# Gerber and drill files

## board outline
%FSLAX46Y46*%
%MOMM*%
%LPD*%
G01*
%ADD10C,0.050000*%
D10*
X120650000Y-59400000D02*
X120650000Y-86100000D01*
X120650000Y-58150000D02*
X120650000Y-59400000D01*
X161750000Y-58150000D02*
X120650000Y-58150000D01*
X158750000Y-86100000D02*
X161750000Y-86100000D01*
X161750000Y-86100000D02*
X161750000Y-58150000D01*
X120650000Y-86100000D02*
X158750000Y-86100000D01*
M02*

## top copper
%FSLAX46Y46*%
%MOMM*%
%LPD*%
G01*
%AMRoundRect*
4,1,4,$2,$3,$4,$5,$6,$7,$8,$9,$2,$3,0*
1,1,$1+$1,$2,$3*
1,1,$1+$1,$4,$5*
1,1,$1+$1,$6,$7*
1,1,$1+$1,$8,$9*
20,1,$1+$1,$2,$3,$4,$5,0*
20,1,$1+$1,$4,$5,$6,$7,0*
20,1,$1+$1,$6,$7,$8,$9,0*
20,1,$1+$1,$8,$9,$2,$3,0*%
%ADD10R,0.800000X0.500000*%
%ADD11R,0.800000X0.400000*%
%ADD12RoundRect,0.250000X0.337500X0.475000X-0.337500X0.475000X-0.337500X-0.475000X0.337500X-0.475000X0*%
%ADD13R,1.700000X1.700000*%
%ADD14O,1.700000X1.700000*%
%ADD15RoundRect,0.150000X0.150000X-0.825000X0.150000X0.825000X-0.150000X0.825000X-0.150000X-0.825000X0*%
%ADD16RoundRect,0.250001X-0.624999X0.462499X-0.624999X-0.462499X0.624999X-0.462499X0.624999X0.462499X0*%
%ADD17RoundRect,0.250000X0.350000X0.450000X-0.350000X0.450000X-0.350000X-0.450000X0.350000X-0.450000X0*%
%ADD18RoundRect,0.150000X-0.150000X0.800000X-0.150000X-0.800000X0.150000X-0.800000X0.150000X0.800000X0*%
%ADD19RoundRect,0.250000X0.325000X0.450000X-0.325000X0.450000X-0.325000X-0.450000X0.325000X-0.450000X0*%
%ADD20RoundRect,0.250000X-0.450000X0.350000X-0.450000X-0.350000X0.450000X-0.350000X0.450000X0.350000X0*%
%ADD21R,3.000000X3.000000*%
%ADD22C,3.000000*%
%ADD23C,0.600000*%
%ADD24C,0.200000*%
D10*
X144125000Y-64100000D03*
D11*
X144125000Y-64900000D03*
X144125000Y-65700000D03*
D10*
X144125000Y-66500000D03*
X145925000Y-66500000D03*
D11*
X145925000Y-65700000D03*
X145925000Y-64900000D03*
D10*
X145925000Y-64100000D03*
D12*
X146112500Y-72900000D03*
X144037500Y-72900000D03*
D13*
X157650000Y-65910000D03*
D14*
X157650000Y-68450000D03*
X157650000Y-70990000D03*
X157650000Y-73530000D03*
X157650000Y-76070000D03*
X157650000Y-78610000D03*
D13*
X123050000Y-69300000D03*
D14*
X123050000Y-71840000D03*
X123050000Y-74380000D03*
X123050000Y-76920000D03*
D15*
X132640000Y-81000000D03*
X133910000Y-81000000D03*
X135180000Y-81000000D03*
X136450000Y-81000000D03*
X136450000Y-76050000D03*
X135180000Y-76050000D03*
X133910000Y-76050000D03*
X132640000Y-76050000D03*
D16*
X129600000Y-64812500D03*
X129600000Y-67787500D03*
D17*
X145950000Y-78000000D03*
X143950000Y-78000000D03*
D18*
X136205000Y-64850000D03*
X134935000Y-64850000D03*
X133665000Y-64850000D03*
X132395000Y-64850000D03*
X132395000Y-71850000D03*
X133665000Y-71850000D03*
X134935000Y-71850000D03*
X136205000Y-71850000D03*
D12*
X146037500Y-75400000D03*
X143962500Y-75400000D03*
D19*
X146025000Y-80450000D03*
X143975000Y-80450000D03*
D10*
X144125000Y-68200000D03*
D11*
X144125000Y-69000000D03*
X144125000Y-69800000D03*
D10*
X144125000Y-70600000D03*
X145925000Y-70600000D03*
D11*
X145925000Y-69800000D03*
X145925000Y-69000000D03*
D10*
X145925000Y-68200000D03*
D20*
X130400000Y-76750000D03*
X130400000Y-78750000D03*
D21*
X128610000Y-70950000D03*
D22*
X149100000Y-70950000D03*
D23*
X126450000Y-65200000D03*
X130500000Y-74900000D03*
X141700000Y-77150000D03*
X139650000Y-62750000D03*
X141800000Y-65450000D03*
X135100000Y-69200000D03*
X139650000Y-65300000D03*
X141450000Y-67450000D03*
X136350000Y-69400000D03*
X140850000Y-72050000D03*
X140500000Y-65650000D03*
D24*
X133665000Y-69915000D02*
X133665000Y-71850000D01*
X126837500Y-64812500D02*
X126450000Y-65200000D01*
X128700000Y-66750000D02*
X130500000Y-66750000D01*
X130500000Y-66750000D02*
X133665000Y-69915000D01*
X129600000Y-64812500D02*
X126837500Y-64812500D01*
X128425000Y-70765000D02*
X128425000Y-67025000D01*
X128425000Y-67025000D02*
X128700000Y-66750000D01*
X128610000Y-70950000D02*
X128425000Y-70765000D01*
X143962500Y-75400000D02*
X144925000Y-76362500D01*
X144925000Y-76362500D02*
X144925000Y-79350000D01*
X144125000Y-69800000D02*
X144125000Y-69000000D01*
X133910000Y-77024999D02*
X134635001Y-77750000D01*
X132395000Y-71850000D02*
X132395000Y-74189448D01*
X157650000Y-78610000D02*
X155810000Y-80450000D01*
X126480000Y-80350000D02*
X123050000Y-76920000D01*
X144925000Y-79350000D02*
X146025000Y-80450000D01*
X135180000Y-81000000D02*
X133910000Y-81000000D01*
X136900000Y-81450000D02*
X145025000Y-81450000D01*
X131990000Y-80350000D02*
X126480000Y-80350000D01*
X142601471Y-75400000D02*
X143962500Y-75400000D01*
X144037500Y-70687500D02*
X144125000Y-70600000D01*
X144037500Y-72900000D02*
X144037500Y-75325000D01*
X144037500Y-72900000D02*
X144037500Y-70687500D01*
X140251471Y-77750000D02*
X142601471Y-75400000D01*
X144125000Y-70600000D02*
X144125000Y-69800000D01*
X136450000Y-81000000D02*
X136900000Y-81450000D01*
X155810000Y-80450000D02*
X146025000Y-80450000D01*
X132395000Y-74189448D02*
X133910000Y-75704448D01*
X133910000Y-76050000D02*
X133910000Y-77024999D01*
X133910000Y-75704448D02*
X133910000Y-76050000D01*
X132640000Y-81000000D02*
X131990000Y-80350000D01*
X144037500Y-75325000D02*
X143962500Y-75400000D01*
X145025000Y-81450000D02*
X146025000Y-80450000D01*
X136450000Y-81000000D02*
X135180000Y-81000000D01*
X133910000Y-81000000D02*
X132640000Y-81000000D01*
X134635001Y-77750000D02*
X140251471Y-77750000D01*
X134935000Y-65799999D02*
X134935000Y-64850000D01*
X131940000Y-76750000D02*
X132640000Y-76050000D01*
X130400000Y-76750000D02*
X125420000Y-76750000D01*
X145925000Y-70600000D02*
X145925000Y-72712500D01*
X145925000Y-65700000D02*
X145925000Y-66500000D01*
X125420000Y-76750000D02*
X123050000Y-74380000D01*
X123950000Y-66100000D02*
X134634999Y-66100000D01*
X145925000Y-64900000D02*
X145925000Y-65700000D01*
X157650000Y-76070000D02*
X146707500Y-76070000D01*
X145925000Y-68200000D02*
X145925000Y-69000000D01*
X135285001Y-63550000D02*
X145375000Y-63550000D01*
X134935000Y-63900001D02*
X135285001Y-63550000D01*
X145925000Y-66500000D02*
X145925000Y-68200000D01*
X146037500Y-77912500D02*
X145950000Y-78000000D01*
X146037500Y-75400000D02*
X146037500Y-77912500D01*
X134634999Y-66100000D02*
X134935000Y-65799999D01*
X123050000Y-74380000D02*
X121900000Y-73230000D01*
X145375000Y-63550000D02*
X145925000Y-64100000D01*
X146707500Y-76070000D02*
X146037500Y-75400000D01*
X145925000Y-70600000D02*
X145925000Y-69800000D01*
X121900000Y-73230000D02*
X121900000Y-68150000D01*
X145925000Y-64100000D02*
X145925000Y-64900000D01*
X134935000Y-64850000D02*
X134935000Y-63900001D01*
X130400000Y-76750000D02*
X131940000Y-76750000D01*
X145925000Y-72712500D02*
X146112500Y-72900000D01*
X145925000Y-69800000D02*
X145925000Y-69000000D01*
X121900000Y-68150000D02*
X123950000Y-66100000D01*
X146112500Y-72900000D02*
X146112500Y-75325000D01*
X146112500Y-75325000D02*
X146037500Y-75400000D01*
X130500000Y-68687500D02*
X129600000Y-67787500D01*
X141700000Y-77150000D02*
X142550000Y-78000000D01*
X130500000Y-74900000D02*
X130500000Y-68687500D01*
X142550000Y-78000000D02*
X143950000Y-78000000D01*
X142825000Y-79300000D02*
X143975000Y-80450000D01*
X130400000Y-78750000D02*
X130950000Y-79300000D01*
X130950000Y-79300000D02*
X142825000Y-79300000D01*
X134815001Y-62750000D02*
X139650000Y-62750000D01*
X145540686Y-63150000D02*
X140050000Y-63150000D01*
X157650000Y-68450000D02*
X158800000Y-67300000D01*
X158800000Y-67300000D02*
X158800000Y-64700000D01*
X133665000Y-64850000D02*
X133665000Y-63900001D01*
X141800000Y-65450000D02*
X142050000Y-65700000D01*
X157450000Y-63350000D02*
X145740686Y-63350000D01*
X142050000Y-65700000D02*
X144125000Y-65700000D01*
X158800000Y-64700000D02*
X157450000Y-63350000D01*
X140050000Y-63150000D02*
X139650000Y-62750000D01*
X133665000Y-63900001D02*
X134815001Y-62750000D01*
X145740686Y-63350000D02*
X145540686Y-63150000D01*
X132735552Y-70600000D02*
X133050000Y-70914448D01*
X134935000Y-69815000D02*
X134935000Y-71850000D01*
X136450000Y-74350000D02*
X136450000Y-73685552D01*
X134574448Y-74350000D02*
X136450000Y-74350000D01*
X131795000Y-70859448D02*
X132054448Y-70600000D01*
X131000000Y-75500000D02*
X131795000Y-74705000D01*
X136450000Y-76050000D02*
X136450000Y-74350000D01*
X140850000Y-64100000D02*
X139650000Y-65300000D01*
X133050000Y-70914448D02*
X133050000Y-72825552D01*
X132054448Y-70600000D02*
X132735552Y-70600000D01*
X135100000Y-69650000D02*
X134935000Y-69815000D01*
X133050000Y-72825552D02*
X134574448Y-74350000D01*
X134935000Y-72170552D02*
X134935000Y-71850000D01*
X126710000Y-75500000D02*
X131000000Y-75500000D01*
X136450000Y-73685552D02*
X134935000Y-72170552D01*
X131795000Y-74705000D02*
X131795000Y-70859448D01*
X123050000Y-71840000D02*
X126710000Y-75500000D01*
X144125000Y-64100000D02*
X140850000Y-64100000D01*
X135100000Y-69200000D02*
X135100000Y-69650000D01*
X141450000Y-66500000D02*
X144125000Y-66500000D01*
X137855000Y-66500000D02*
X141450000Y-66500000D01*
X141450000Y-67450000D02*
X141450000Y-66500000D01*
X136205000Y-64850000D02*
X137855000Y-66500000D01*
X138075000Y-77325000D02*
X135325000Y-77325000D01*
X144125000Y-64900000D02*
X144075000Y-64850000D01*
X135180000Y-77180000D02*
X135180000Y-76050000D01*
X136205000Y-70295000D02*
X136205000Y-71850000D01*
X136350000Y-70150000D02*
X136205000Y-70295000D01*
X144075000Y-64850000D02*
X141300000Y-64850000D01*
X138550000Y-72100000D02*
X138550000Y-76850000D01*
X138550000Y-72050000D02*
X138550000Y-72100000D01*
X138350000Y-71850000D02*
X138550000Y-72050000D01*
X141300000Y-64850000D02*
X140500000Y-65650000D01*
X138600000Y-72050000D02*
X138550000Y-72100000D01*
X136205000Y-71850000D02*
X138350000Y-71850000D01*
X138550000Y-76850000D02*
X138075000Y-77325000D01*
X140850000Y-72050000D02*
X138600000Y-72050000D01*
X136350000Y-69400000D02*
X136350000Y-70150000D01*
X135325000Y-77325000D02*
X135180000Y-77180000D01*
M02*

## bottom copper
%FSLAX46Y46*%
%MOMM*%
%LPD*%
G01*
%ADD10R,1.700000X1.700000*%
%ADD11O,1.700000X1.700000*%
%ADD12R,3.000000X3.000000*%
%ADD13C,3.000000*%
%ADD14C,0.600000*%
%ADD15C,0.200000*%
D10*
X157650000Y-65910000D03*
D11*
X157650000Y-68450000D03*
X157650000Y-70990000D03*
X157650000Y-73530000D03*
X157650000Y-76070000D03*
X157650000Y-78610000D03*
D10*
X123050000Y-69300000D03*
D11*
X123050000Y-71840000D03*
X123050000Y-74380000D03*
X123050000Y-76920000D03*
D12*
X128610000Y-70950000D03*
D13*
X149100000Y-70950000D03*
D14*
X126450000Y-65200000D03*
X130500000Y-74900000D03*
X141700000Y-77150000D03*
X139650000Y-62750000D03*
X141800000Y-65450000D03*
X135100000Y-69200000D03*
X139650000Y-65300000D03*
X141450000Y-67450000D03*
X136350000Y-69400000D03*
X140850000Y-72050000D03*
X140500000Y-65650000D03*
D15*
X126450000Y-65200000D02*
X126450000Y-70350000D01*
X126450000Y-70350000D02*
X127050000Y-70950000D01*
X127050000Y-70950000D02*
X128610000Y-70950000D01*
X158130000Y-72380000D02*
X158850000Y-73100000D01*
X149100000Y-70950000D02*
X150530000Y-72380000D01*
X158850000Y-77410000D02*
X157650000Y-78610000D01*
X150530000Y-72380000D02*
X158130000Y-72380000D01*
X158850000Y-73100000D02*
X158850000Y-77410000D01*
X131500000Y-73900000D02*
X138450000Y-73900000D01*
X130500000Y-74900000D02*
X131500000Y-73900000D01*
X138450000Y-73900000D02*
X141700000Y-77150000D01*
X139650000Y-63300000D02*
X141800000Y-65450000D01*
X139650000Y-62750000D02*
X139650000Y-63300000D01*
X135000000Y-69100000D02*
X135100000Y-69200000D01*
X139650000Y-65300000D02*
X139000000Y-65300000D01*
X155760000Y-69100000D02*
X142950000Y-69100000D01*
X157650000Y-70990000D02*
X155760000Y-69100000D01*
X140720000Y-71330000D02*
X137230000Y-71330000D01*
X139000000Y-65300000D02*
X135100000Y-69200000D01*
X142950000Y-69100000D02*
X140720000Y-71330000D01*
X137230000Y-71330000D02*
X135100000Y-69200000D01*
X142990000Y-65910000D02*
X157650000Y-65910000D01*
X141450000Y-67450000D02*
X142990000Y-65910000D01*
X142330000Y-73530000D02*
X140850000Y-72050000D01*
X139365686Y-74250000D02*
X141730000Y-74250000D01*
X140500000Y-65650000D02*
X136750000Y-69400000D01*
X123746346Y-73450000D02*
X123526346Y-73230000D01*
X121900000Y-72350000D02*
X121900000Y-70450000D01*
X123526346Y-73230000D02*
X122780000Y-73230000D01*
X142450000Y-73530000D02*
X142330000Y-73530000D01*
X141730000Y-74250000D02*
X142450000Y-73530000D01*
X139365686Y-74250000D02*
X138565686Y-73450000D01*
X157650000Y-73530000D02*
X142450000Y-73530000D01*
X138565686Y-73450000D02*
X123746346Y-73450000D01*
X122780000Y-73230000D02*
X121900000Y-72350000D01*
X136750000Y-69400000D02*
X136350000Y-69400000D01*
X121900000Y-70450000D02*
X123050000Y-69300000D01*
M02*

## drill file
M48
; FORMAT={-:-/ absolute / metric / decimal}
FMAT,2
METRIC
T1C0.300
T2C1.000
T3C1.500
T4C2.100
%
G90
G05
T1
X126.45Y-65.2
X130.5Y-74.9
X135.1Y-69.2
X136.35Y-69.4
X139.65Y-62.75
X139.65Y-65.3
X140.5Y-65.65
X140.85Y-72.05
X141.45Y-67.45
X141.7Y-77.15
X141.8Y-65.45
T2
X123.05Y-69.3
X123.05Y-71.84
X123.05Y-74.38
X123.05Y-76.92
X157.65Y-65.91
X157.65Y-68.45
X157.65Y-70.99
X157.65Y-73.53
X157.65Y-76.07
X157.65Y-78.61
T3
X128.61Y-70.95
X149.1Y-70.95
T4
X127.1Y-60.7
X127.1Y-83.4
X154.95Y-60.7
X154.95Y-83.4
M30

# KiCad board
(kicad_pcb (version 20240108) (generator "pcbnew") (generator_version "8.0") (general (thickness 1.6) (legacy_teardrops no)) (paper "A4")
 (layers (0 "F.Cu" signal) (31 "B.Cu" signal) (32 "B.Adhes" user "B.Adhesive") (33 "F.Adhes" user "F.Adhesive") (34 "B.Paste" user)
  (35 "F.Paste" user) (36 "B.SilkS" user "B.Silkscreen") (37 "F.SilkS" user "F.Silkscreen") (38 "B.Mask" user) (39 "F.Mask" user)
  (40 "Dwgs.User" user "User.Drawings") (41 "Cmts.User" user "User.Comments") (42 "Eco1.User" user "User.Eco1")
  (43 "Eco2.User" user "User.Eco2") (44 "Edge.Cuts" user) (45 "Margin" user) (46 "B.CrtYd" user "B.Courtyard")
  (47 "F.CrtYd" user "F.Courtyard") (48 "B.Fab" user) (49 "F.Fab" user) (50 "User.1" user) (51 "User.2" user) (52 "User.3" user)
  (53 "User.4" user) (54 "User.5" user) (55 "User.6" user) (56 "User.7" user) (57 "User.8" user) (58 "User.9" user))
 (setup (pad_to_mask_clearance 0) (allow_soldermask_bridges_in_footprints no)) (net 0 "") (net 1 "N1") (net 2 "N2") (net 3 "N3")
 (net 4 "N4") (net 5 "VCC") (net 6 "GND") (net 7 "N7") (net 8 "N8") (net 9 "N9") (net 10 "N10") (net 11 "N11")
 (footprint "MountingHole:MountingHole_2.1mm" (layer "F.Cu") (at 127.1 60.7)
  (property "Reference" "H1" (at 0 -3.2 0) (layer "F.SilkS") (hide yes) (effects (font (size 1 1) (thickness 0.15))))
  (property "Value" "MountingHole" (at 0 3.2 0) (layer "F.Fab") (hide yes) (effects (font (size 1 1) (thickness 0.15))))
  (pad "" np_thru_hole circle (at 0 0) (size 2.1 2.1) (drill 2.1) (layers "*.Cu" "*.Mask")))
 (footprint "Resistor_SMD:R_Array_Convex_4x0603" (layer "F.Cu") (at 145.025 65.3)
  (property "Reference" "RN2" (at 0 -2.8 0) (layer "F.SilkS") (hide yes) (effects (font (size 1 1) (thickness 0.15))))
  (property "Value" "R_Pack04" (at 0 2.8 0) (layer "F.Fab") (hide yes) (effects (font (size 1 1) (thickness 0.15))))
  (pad "1" smd rect (at -0.9 -1.2) (size 0.8 0.5) (layers "F.Cu" "F.Paste" "F.Mask") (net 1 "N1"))
  (pad "2" smd rect (at -0.9 -0.4) (size 0.8 0.4) (layers "F.Cu" "F.Paste" "F.Mask") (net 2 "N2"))
  (pad "3" smd rect (at -0.9 0.4) (size 0.8 0.4) (layers "F.Cu" "F.Paste" "F.Mask") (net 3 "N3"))
  (pad "4" smd rect (at -0.9 1.2) (size 0.8 0.5) (layers "F.Cu" "F.Paste" "F.Mask") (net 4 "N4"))
  (pad "5" smd rect (at 0.9 1.2) (size 0.8 0.5) (layers "F.Cu" "F.Paste" "F.Mask") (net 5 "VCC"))
  (pad "6" smd rect (at 0.9 0.4) (size 0.8 0.4) (layers "F.Cu" "F.Paste" "F.Mask") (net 5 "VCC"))
  (pad "7" smd rect (at 0.9 -0.4) (size 0.8 0.4) (layers "F.Cu" "F.Paste" "F.Mask") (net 5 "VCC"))
  (pad "8" smd rect (at 0.9 -1.2) (size 0.8 0.5) (layers "F.Cu" "F.Paste" "F.Mask") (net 5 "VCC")))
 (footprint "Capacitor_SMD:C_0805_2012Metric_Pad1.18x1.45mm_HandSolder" (layer "F.Cu") (at 145.075 72.9 180)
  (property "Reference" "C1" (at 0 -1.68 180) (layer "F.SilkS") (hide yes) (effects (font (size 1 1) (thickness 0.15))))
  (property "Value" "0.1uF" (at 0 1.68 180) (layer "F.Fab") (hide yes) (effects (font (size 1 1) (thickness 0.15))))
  (pad "1" smd roundrect (at -1.0375 0 180) (size 1.175 1.45) (layers "F.Cu" "F.Paste" "F.Mask") (roundrect_rratio 0.212766) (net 5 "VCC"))
  (pad "2" smd roundrect (at 1.0375 0 180) (size 1.175 1.45) (layers "F.Cu" "F.Paste" "F.Mask") (roundrect_rratio 0.212766) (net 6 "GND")))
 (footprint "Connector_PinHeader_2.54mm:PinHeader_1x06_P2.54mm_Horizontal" (layer "F.Cu") (at 157.65 65.91)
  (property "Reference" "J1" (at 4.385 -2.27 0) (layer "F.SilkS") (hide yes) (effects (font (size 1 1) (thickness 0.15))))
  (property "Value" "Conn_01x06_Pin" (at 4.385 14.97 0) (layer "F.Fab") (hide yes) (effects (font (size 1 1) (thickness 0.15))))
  (pad "1" thru_hole rect (at 0 0) (size 1.7 1.7) (drill 1) (layers "*.Cu" "*.Mask") (remove_unused_layers no) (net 4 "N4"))
  (pad "2" thru_hole oval (at 0 2.54) (size 1.7 1.7) (drill 1) (layers "*.Cu" "*.Mask") (remove_unused_layers no) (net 3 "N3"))
  (pad "3" thru_hole oval (at 0 5.08) (size 1.7 1.7) (drill 1) (layers "*.Cu" "*.Mask") (remove_unused_layers no) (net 1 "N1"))
  (pad "4" thru_hole oval (at 0 7.62) (size 1.7 1.7) (drill 1) (layers "*.Cu" "*.Mask") (remove_unused_layers no) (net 2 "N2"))
  (pad "5" thru_hole oval (at 0 10.16) (size 1.7 1.7) (drill 1) (layers "*.Cu" "*.Mask") (remove_unused_layers no) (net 5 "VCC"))
  (pad "6" thru_hole oval (at 0 12.7) (size 1.7 1.7) (drill 1) (layers "*.Cu" "*.Mask") (remove_unused_layers no) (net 6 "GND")))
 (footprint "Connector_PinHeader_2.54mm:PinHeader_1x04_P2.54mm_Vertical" (layer "F.Cu") (at 123.05 69.3)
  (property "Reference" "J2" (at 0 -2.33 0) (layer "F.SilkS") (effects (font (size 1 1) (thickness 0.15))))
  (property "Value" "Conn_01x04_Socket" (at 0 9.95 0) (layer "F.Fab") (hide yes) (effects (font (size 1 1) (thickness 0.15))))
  (pad "1" thru_hole rect (at 0 0) (size 1.7 1.7) (drill 1) (layers "*.Cu" "*.Mask") (remove_unused_layers no) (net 2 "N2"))
  (pad "2" thru_hole oval (at 0 2.54) (size 1.7 1.7) (drill 1) (layers "*.Cu" "*.Mask") (remove_unused_layers no) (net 1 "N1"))
  (pad "3" thru_hole oval (at 0 5.08) (size 1.7 1.7) (drill 1) (layers "*.Cu" "*.Mask") (remove_unused_layers no) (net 5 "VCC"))
  (pad "4" thru_hole oval (at 0 7.62) (size 1.7 1.7) (drill 1) (layers "*.Cu" "*.Mask") (remove_unused_layers no) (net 6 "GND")))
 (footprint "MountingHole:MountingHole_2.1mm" (layer "F.Cu") (at 154.95 60.7)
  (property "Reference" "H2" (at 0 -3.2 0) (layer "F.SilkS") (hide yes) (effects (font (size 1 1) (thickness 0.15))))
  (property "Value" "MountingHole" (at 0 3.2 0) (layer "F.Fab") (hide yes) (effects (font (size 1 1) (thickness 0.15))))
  (pad "" np_thru_hole circle (at 0 0) (size 2.1 2.1) (drill 2.1) (layers "*.Cu" "*.Mask")))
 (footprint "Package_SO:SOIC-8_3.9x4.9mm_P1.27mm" (layer "F.Cu") (at 134.545 78.525 90)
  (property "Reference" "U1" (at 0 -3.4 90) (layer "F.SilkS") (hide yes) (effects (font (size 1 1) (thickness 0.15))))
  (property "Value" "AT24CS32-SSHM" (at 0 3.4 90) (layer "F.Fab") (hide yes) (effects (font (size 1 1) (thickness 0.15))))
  (pad "1" smd roundrect (at -2.475 -1.905 90) (size 1.95 0.6) (layers "F.Cu" "F.Paste" "F.Mask") (roundrect_rratio 0.25) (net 6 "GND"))
  (pad "2" smd roundrect (at -2.475 -0.635 90) (size 1.95 0.6) (layers "F.Cu" "F.Paste" "F.Mask") (roundrect_rratio 0.25) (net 6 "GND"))
  (pad "3" smd roundrect (at -2.475 0.635 90) (size 1.95 0.6) (layers "F.Cu" "F.Paste" "F.Mask") (roundrect_rratio 0.25) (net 6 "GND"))
  (pad "4" smd roundrect (at -2.475 1.905 90) (size 1.95 0.6) (layers "F.Cu" "F.Paste" "F.Mask") (roundrect_rratio 0.25) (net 6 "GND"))
  (pad "5" smd roundrect (at 2.475 1.905 90) (size 1.95 0.6) (layers "F.Cu" "F.Paste" "F.Mask") (roundrect_rratio 0.25) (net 1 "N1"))
  (pad "6" smd roundrect (at 2.475 0.635 90) (size 1.95 0.6) (layers "F.Cu" "F.Paste" "F.Mask") (roundrect_rratio 0.25) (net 2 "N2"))
  (pad "7" smd roundrect (at 2.475 -0.635 90) (size 1.95 0.6) (layers "F.Cu" "F.Paste" "F.Mask") (roundrect_rratio 0.25) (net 6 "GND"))
  (pad "8" smd roundrect (at 2.475 -1.905 90) (size 1.95 0.6) (layers "F.Cu" "F.Paste" "F.Mask") (roundrect_rratio 0.25) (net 5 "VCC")))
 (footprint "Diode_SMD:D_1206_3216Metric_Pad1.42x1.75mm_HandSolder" (layer "F.Cu") (at 129.6 66.3 -90)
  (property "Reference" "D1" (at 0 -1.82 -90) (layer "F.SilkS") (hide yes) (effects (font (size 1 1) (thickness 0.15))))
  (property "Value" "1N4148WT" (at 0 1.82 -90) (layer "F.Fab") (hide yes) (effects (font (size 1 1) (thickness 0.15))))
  (pad "1" smd roundrect (at -1.4875 0 270) (size 1.425 1.75) (layers "F.Cu" "F.Paste" "F.Mask") (roundrect_rratio 0.175439) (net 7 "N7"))
  (pad "2" smd roundrect (at 1.4875 0 270) (size 1.425 1.75) (layers "F.Cu" "F.Paste" "F.Mask") (roundrect_rratio 0.175439) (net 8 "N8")))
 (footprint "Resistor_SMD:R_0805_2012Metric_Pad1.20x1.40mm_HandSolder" (layer "F.Cu") (at 144.95 78 180)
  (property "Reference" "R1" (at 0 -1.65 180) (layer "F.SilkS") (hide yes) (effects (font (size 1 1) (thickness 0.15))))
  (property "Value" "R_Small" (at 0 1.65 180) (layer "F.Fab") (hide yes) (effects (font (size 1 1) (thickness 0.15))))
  (pad "1" smd roundrect (at -1 0 180) (size 1.2 1.4) (layers "F.Cu" "F.Paste" "F.Mask") (roundrect_rratio 0.208333) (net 5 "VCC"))
  (pad "2" smd roundrect (at 1 0 180) (size 1.2 1.4) (layers "F.Cu" "F.Paste" "F.Mask") (roundrect_rratio 0.208333) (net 8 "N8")))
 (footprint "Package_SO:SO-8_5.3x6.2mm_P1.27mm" (layer "F.Cu") (at 134.3 68.35 -90)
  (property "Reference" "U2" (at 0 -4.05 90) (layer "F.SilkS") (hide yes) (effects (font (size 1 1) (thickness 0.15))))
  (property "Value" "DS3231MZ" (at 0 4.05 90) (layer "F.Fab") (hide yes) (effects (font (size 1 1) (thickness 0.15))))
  (pad "1" smd roundrect (at -3.5 -1.905 270) (size 1.9 0.6) (layers "F.Cu" "F.Paste" "F.Mask") (roundrect_rratio 0.25) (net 4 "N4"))
  (pad "2" smd roundrect (at -3.5 -0.635 270) (size 1.9 0.6) (layers "F.Cu" "F.Paste" "F.Mask") (roundrect_rratio 0.25) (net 5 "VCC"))
  (pad "3" smd roundrect (at -3.5 0.635 270) (size 1.9 0.6) (layers "F.Cu" "F.Paste" "F.Mask") (roundrect_rratio 0.25) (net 3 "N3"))
  (pad "4" smd roundrect (at -3.5 1.905 270) (size 1.9 0.6) (layers "F.Cu" "F.Paste" "F.Mask") (roundrect_rratio 0.25) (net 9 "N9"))
  (pad "5" smd roundrect (at 3.5 1.905 270) (size 1.9 0.6) (layers "F.Cu" "F.Paste" "F.Mask") (roundrect_rratio 0.25) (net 6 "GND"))
  (pad "6" smd roundrect (at 3.5 0.635 270) (size 1.9 0.6) (layers "F.Cu" "F.Paste" "F.Mask") (roundrect_rratio 0.25) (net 7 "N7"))
  (pad "7" smd roundrect (at 3.5 -0.635 270) (size 1.9 0.6) (layers "F.Cu" "F.Paste" "F.Mask") (roundrect_rratio 0.25) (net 1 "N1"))
  (pad "8" smd roundrect (at 3.5 -1.905 270) (size 1.9 0.6) (layers "F.Cu" "F.Paste" "F.Mask") (roundrect_rratio 0.25) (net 2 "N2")))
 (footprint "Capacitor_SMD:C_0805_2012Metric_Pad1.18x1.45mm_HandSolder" (layer "F.Cu") (at 145 75.4 180)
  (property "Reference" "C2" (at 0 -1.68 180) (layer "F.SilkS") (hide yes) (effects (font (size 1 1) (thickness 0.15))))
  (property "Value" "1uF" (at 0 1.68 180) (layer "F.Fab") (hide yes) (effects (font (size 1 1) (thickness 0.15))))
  (pad "1" smd roundrect (at -1.0375 0 180) (size 1.175 1.45) (layers "F.Cu" "F.Paste" "F.Mask") (roundrect_rratio 0.212766) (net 5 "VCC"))
  (pad "2" smd roundrect (at 1.0375 0 180) (size 1.175 1.45) (layers "F.Cu" "F.Paste" "F.Mask") (roundrect_rratio 0.212766) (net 6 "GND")))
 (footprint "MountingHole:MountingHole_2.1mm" (layer "F.Cu") (at 154.95 83.4)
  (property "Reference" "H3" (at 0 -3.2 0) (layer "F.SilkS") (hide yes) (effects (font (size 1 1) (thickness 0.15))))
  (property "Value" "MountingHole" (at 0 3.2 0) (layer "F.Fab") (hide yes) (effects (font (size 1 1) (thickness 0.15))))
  (pad "" np_thru_hole circle (at 0 0) (size 2.1 2.1) (drill 2.1) (layers "*.Cu" "*.Mask")))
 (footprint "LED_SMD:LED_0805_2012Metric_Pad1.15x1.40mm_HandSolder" (layer "F.Cu") (at 145 80.45 180)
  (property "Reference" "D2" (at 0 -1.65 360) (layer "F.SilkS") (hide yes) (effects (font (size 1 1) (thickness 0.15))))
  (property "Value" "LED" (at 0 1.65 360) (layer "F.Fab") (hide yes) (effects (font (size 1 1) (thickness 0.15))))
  (pad "1" smd roundrect (at -1.025 0 180) (size 1.15 1.4) (layers "F.Cu" "F.Paste" "F.Mask") (roundrect_rratio 0.217391) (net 6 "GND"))
  (pad "2" smd roundrect (at 1.025 0 180) (size 1.15 1.4) (layers "F.Cu" "F.Paste" "F.Mask") (roundrect_rratio 0.217391) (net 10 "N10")))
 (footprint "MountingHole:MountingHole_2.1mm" (layer "F.Cu") (at 127.1 83.4)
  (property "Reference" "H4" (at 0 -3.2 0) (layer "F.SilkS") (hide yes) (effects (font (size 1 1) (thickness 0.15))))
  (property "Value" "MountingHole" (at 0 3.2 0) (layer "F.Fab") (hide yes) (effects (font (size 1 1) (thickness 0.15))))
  (pad "" np_thru_hole circle (at 0 0) (size 2.1 2.1) (drill 2.1) (layers "*.Cu" "*.Mask")))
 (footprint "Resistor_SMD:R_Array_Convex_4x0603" (layer "F.Cu") (at 145.025 69.4)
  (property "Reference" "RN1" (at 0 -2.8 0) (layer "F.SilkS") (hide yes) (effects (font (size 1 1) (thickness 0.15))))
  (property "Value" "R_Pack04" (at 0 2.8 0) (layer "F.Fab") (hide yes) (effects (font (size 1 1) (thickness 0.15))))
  (pad "1" smd rect (at -0.9 -1.2) (size 0.8 0.5) (layers "F.Cu" "F.Paste" "F.Mask") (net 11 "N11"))
  (pad "2" smd rect (at -0.9 -0.4) (size 0.8 0.4) (layers "F.Cu" "F.Paste" "F.Mask") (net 6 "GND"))
  (pad "3" smd rect (at -0.9 0.4) (size 0.8 0.4) (layers "F.Cu" "F.Paste" "F.Mask") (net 6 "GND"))
  (pad "4" smd rect (at -0.9 1.2) (size 0.8 0.5) (layers "F.Cu" "F.Paste" "F.Mask") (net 6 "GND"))
  (pad "5" smd rect (at 0.9 1.2) (size 0.8 0.5) (layers "F.Cu" "F.Paste" "F.Mask") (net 5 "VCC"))
  (pad "6" smd rect (at 0.9 0.4) (size 0.8 0.4) (layers "F.Cu" "F.Paste" "F.Mask") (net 5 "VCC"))
  (pad "7" smd rect (at 0.9 -0.4) (size 0.8 0.4) (layers "F.Cu" "F.Paste" "F.Mask") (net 5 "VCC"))
  (pad "8" smd rect (at 0.9 -1.2) (size 0.8 0.5) (layers "F.Cu" "F.Paste" "F.Mask") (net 5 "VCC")))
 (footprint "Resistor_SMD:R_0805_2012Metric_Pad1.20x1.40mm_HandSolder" (layer "F.Cu") (at 130.4 77.75 -90)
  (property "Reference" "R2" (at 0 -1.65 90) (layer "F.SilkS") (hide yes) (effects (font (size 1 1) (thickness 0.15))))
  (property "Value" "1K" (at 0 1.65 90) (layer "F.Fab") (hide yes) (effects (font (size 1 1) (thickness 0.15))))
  (pad "1" smd roundrect (at -1 0 270) (size 1.2 1.4) (layers "F.Cu" "F.Paste" "F.Mask") (roundrect_rratio 0.208333) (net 5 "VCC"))
  (pad "2" smd roundrect (at 1 0 270) (size 1.2 1.4) (layers "F.Cu" "F.Paste" "F.Mask") (roundrect_rratio 0.208333) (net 10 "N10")))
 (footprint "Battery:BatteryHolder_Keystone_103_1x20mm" (layer "B.Cu") (at 128.61 70.95)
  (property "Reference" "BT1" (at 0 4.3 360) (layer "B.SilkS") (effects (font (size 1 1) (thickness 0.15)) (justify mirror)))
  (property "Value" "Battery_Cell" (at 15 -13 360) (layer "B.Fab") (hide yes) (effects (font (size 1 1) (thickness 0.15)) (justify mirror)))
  (pad "1" thru_hole rect (at 0 0) (size 3 3) (drill 1.5) (layers "*.Cu" "*.Mask") (remove_unused_layers no) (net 7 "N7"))
  (pad "2" thru_hole circle (at 20.49 0) (size 3 3) (drill 1.5) (layers "*.Cu" "*.Mask") (remove_unused_layers no) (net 6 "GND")))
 (gr_line (start 120.65 59.4) (end 120.65 86.1) (stroke (width 0.05) (type default)) (layer "Edge.Cuts"))
 (gr_line (start 120.65 58.15) (end 120.65 59.4) (stroke (width 0.05) (type default)) (layer "Edge.Cuts"))
 (gr_line (start 161.75 58.15) (end 120.65 58.15) (stroke (width 0.05) (type default)) (layer "Edge.Cuts"))
 (gr_line (start 158.75 86.1) (end 161.75 86.1) (stroke (width 0.05) (type default)) (layer "Edge.Cuts"))
 (gr_line (start 161.75 86.1) (end 161.75 58.15) (stroke (width 0.05) (type default)) (layer "Edge.Cuts"))
 (gr_line (start 120.65 86.1) (end 158.75 86.1) (stroke (width 0.05) (type default)) (layer "Edge.Cuts"))
 (segment (start 133.665 69.915) (end 133.665 71.85) (width 0.2) (layer "F.Cu") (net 7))
 (segment (start 126.8375 64.8125) (end 126.45 65.2) (width 0.2) (layer "F.Cu") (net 7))
 (segment (start 128.7 66.75) (end 130.5 66.75) (width 0.2) (layer "F.Cu") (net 7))
 (segment (start 130.5 66.75) (end 133.665 69.915) (width 0.2) (layer "F.Cu") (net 7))
 (segment (start 129.6 64.8125) (end 126.8375 64.8125) (width 0.2) (layer "F.Cu") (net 7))
 (segment (start 128.425 70.765) (end 128.425 67.025) (width 0.2) (layer "F.Cu") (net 7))
 (segment (start 128.425 67.025) (end 128.7 66.75) (width 0.2) (layer "F.Cu") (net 7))
 (segment (start 128.61 70.95) (end 128.425 70.765) (width 0.2) (layer "F.Cu") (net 7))
 (via (at 126.45 65.2) (size 0.6) (drill 0.3) (layers "F.Cu" "B.Cu") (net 7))
 (segment (start 126.45 65.2) (end 126.45 70.35) (width 0.2) (layer "B.Cu") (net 7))
 (segment (start 126.45 70.35) (end 127.05 70.95) (width 0.2) (layer "B.Cu") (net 7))
 (segment (start 127.05 70.95) (end 128.61 70.95) (width 0.2) (layer "B.Cu") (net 7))
 (segment (start 143.9625 75.4) (end 144.925 76.3625) (width 0.2) (layer "F.Cu") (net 6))
 (segment (start 144.925 76.3625) (end 144.925 79.35) (width 0.2) (layer "F.Cu") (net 6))
 (segment (start 144.125 69.8) (end 144.125 69) (width 0.2) (layer "F.Cu") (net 6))
 (segment (start 133.91 77.024999) (end 134.635001 77.75) (width 0.2) (layer "F.Cu") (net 6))
 (segment (start 132.395 71.85) (end 132.395 74.189448) (width 0.2) (layer "F.Cu") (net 6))
 (segment (start 157.65 78.61) (end 155.81 80.45) (width 0.2) (layer "F.Cu") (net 6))
 (segment (start 126.48 80.35) (end 123.05 76.92) (width 0.2) (layer "F.Cu") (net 6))
 (segment (start 144.925 79.35) (end 146.025 80.45) (width 0.2) (layer "F.Cu") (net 6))
 (segment (start 135.18 81) (end 133.91 81) (width 0.2) (layer "F.Cu") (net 6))
 (segment (start 136.9 81.45) (end 145.025 81.45) (width 0.2) (layer "F.Cu") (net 6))
 (segment (start 131.99 80.35) (end 126.48 80.35) (width 0.2) (layer "F.Cu") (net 6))
 (segment (start 142.601471 75.4) (end 143.9625 75.4) (width 0.2) (layer "F.Cu") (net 6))
 (segment (start 144.0375 70.6875) (end 144.125 70.6) (width 0.2) (layer "F.Cu") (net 6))
 (segment (start 144.0375 72.9) (end 144.0375 75.325) (width 0.2) (layer "F.Cu") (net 6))
 (segment (start 144.0375 72.9) (end 144.0375 70.6875) (width 0.2) (layer "F.Cu") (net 6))
 (segment (start 140.251471 77.75) (end 142.601471 75.4) (width 0.2) (layer "F.Cu") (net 6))
 (segment (start 144.125 70.6) (end 144.125 69.8) (width 0.2) (layer "F.Cu") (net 6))
 (segment (start 136.45 81) (end 136.9 81.45) (width 0.2) (layer "F.Cu") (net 6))
 (segment (start 155.81 80.45) (end 146.025 80.45) (width 0.2) (layer "F.Cu") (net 6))
 (segment (start 132.395 74.189448) (end 133.91 75.704448) (width 0.2) (layer "F.Cu") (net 6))
 (segment (start 133.91 76.05) (end 133.91 77.024999) (width 0.2) (layer "F.Cu") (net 6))
 (segment (start 133.91 75.704448) (end 133.91 76.05) (width 0.2) (layer "F.Cu") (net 6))
 (segment (start 132.64 81) (end 131.99 80.35) (width 0.2) (layer "F.Cu") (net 6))
 (segment (start 144.0375 75.325) (end 143.9625 75.4) (width 0.2) (layer "F.Cu") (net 6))
 (segment (start 145.025 81.45) (end 146.025 80.45) (width 0.2) (layer "F.Cu") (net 6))
 (segment (start 136.45 81) (end 135.18 81) (width 0.2) (layer "F.Cu") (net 6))
 (segment (start 133.91 81) (end 132.64 81) (width 0.2) (layer "F.Cu") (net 6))
 (segment (start 134.635001 77.75) (end 140.251471 77.75) (width 0.2) (layer "F.Cu") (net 6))
 (segment (start 158.13 72.38) (end 158.85 73.1) (width 0.2) (layer "B.Cu") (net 6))
 (segment (start 149.1 70.95) (end 150.53 72.38) (width 0.2) (layer "B.Cu") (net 6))
 (segment (start 158.85 77.41) (end 157.65 78.61) (width 0.2) (layer "B.Cu") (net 6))
 (segment (start 150.53 72.38) (end 158.13 72.38) (width 0.2) (layer "B.Cu") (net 6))
 (segment (start 158.85 73.1) (end 158.85 77.41) (width 0.2) (layer "B.Cu") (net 6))
 (segment (start 134.935 65.799999) (end 134.935 64.85) (width 0.2) (layer "F.Cu") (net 5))
 (segment (start 131.94 76.75) (end 132.64 76.05) (width 0.2) (layer "F.Cu") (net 5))
 (segment (start 130.4 76.75) (end 125.42 76.75) (width 0.2) (layer "F.Cu") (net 5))
 (segment (start 145.925 70.6) (end 145.925 72.7125) (width 0.2) (layer "F.Cu") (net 5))
 (segment (start 145.925 65.7) (end 145.925 66.5) (width 0.2) (layer "F.Cu") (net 5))
 (segment (start 125.42 76.75) (end 123.05 74.38) (width 0.2) (layer "F.Cu") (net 5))
 (segment (start 123.95 66.1) (end 134.634999 66.1) (width 0.2) (layer "F.Cu") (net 5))
 (segment (start 145.925 64.9) (end 145.925 65.7) (width 0.2) (layer "F.Cu") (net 5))
 (segment (start 157.65 76.07) (end 146.7075 76.07) (width 0.2) (layer "F.Cu") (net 5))
 (segment (start 145.925 68.2) (end 145.925 69) (width 0.2) (layer "F.Cu") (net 5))
 (segment (start 135.285001 63.55) (end 145.375 63.55) (width 0.2) (layer "F.Cu") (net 5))
 (segment (start 134.935 63.900001) (end 135.285001 63.55) (width 0.2) (layer "F.Cu") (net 5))
 (segment (start 145.925 66.5) (end 145.925 68.2) (width 0.2) (layer "F.Cu") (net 5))
 (segment (start 146.0375 77.9125) (end 145.95 78) (width 0.2) (layer "F.Cu") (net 5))
 (segment (start 146.0375 75.4) (end 146.0375 77.9125) (width 0.2) (layer "F.Cu") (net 5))
 (segment (start 134.634999 66.1) (end 134.935 65.799999) (width 0.2) (layer "F.Cu") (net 5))
 (segment (start 123.05 74.38) (end 121.9 73.23) (width 0.2) (layer "F.Cu") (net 5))
 (segment (start 145.375 63.55) (end 145.925 64.1) (width 0.2) (layer "F.Cu") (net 5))
 (segment (start 146.7075 76.07) (end 146.0375 75.4) (width 0.2) (layer "F.Cu") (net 5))
 (segment (start 145.925 70.6) (end 145.925 69.8) (width 0.2) (layer "F.Cu") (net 5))
 (segment (start 121.9 73.23) (end 121.9 68.15) (width 0.2) (layer "F.Cu") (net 5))
 (segment (start 145.925 64.1) (end 145.925 64.9) (width 0.2) (layer "F.Cu") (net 5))
 (segment (start 134.935 64.85) (end 134.935 63.900001) (width 0.2) (layer "F.Cu") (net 5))
 (segment (start 130.4 76.75) (end 131.94 76.75) (width 0.2) (layer "F.Cu") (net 5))
 (segment (start 145.925 72.7125) (end 146.1125 72.9) (width 0.2) (layer "F.Cu") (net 5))
 (segment (start 145.925 69.8) (end 145.925 69) (width 0.2) (layer "F.Cu") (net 5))
 (segment (start 121.9 68.15) (end 123.95 66.1) (width 0.2) (layer "F.Cu") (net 5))
 (segment (start 146.1125 72.9) (end 146.1125 75.325) (width 0.2) (layer "F.Cu") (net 5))
 (segment (start 146.1125 75.325) (end 146.0375 75.4) (width 0.2) (layer "F.Cu") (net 5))
 (segment (start 130.5 68.6875) (end 129.6 67.7875) (width 0.2) (layer "F.Cu") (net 8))
 (segment (start 141.7 77.15) (end 142.55 78) (width 0.2) (layer "F.Cu") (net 8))
 (segment (start 130.5 74.9) (end 130.5 68.6875) (width 0.2) (layer "F.Cu") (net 8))
 (segment (start 142.55 78) (end 143.95 78) (width 0.2) (layer "F.Cu") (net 8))
 (via (at 130.5 74.9) (size 0.6) (drill 0.3) (layers "F.Cu" "B.Cu") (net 8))
 (via (at 141.7 77.15) (size 0.6) (drill 0.3) (layers "F.Cu" "B.Cu") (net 8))
 (segment (start 131.5 73.9) (end 138.45 73.9) (width 0.2) (layer "B.Cu") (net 8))
 (segment (start 130.5 74.9) (end 131.5 73.9) (width 0.2) (layer "B.Cu") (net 8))
 (segment (start 138.45 73.9) (end 141.7 77.15) (width 0.2) (layer "B.Cu") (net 8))
 (segment (start 142.825 79.3) (end 143.975 80.45) (width 0.2) (layer "F.Cu") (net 10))
 (segment (start 130.4 78.75) (end 130.95 79.3) (width 0.2) (layer "F.Cu") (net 10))
 (segment (start 130.95 79.3) (end 142.825 79.3) (width 0.2) (layer "F.Cu") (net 10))
 (segment (start 134.815001 62.75) (end 139.65 62.75) (width 0.2) (layer "F.Cu") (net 3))
 (segment (start 145.540686 63.15) (end 140.05 63.15) (width 0.2) (layer "F.Cu") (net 3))
 (segment (start 157.65 68.45) (end 158.8 67.3) (width 0.2) (layer "F.Cu") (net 3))
 (segment (start 158.8 67.3) (end 158.8 64.7) (width 0.2) (layer "F.Cu") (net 3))
 (segment (start 133.665 64.85) (end 133.665 63.900001) (width 0.2) (layer "F.Cu") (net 3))
 (segment (start 141.8 65.45) (end 142.05 65.7) (width 0.2) (layer "F.Cu") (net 3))
 (segment (start 157.45 63.35) (end 145.740686 63.35) (width 0.2) (layer "F.Cu") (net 3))
 (segment (start 142.05 65.7) (end 144.125 65.7) (width 0.2) (layer "F.Cu") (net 3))
 (segment (start 158.8 64.7) (end 157.45 63.35) (width 0.2) (layer "F.Cu") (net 3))
 (segment (start 140.05 63.15) (end 139.65 62.75) (width 0.2) (layer "F.Cu") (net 3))
 (segment (start 133.665 63.900001) (end 134.815001 62.75) (width 0.2) (layer "F.Cu") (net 3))
 (segment (start 145.740686 63.35) (end 145.540686 63.15) (width 0.2) (layer "F.Cu") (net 3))
 (via (at 139.65 62.75) (size 0.6) (drill 0.3) (layers "F.Cu" "B.Cu") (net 3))
 (via (at 141.8 65.45) (size 0.6) (drill 0.3) (layers "F.Cu" "B.Cu") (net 3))
 (segment (start 139.65 63.3) (end 141.8 65.45) (width 0.2) (layer "B.Cu") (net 3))
 (segment (start 139.65 62.75) (end 139.65 63.3) (width 0.2) (layer "B.Cu") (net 3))
 (segment (start 132.735552 70.6) (end 133.05 70.914448) (width 0.2) (layer "F.Cu") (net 1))
 (segment (start 134.935 69.815) (end 134.935 71.85) (width 0.2) (layer "F.Cu") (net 1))
 (segment (start 136.45 74.35) (end 136.45 73.685552) (width 0.2) (layer "F.Cu") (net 1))
 (segment (start 134.574448 74.35) (end 136.45 74.35) (width 0.2) (layer "F.Cu") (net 1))
 (segment (start 131.795 70.859448) (end 132.054448 70.6) (width 0.2) (layer "F.Cu") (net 1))
 (segment (start 131 75.5) (end 131.795 74.705) (width 0.2) (layer "F.Cu") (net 1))
 (segment (start 136.45 76.05) (end 136.45 74.35) (width 0.2) (layer "F.Cu") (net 1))
 (segment (start 140.85 64.1) (end 139.65 65.3) (width 0.2) (layer "F.Cu") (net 1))
 (segment (start 133.05 70.914448) (end 133.05 72.825552) (width 0.2) (layer "F.Cu") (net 1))
 (segment (start 132.054448 70.6) (end 132.735552 70.6) (width 0.2) (layer "F.Cu") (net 1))
 (segment (start 135.1 69.65) (end 134.935 69.815) (width 0.2) (layer "F.Cu") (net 1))
 (segment (start 133.05 72.825552) (end 134.574448 74.35) (width 0.2) (layer "F.Cu") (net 1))
 (segment (start 134.935 72.170552) (end 134.935 71.85) (width 0.2) (layer "F.Cu") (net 1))
 (segment (start 126.71 75.5) (end 131 75.5) (width 0.2) (layer "F.Cu") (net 1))
 (segment (start 136.45 73.685552) (end 134.935 72.170552) (width 0.2) (layer "F.Cu") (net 1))
 (segment (start 131.795 74.705) (end 131.795 70.859448) (width 0.2) (layer "F.Cu") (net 1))
 (segment (start 123.05 71.84) (end 126.71 75.5) (width 0.2) (layer "F.Cu") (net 1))
 (segment (start 144.125 64.1) (end 140.85 64.1) (width 0.2) (layer "F.Cu") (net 1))
 (segment (start 135.1 69.2) (end 135.1 69.65) (width 0.2) (layer "F.Cu") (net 1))
 (via (at 135.1 69.2) (size 0.6) (drill 0.3) (layers "F.Cu" "B.Cu") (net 1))
 (via (at 139.65 65.3) (size 0.6) (drill 0.3) (layers "F.Cu" "B.Cu") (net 1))
 (segment (start 135 69.1) (end 135.1 69.2) (width 0.2) (layer "B.Cu") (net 1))
 (segment (start 139.65 65.3) (end 139 65.3) (width 0.2) (layer "B.Cu") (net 1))
 (segment (start 155.76 69.1) (end 142.95 69.1) (width 0.2) (layer "B.Cu") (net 1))
 (segment (start 157.65 70.99) (end 155.76 69.1) (width 0.2) (layer "B.Cu") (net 1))
 (segment (start 140.72 71.33) (end 137.23 71.33) (width 0.2) (layer "B.Cu") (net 1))
 (segment (start 139 65.3) (end 135.1 69.2) (width 0.2) (layer "B.Cu") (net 1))
 (segment (start 142.95 69.1) (end 140.72 71.33) (width 0.2) (layer "B.Cu") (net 1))
 (segment (start 137.23 71.33) (end 135.1 69.2) (width 0.2) (layer "B.Cu") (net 1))
 (segment (start 141.45 66.5) (end 144.125 66.5) (width 0.2) (layer "F.Cu") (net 4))
 (segment (start 137.855 66.5) (end 141.45 66.5) (width 0.2) (layer "F.Cu") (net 4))
 (segment (start 141.45 67.45) (end 141.45 66.5) (width 0.2) (layer "F.Cu") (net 4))
 (segment (start 136.205 64.85) (end 137.855 66.5) (width 0.2) (layer "F.Cu") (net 4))
 (via (at 141.45 67.45) (size 0.6) (drill 0.3) (layers "F.Cu" "B.Cu") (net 4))
 (segment (start 142.99 65.91) (end 157.65 65.91) (width 0.2) (layer "B.Cu") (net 4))
 (segment (start 141.45 67.45) (end 142.99 65.91) (width 0.2) (layer "B.Cu") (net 4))
 (segment (start 138.075 77.325) (end 135.325 77.325) (width 0.2) (layer "F.Cu") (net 2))
 (segment (start 144.125 64.9) (end 144.075 64.85) (width 0.2) (layer "F.Cu") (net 2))
 (segment (start 135.18 77.18) (end 135.18 76.05) (width 0.2) (layer "F.Cu") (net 2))
 (segment (start 136.205 70.295) (end 136.205 71.85) (width 0.2) (layer "F.Cu") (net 2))
 (segment (start 136.35 70.15) (end 136.205 70.295) (width 0.2) (layer "F.Cu") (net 2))
 (segment (start 144.075 64.85) (end 141.3 64.85) (width 0.2) (layer "F.Cu") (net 2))
 (segment (start 138.55 72.1) (end 138.55 76.85) (width 0.2) (layer "F.Cu") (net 2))
 (segment (start 138.55 72.05) (end 138.55 72.1) (width 0.2) (layer "F.Cu") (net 2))
 (segment (start 138.35 71.85) (end 138.55 72.05) (width 0.2) (layer "F.Cu") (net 2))
 (segment (start 141.3 64.85) (end 140.5 65.65) (width 0.2) (layer "F.Cu") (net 2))
 (segment (start 138.6 72.05) (end 138.55 72.1) (width 0.2) (layer "F.Cu") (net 2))
 (segment (start 136.205 71.85) (end 138.35 71.85) (width 0.2) (layer "F.Cu") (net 2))
 (segment (start 138.55 76.85) (end 138.075 77.325) (width 0.2) (layer "F.Cu") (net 2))
 (segment (start 140.85 72.05) (end 138.6 72.05) (width 0.2) (layer "F.Cu") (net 2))
 (segment (start 136.35 69.4) (end 136.35 70.15) (width 0.2) (layer "F.Cu") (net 2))
 (segment (start 135.325 77.325) (end 135.18 77.18) (width 0.2) (layer "F.Cu") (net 2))
 (via (at 136.35 69.4) (size 0.6) (drill 0.3) (layers "F.Cu" "B.Cu") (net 2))
 (via (at 140.85 72.05) (size 0.6) (drill 0.3) (layers "F.Cu" "B.Cu") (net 2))
 (via (at 140.5 65.65) (size 0.6) (drill 0.3) (layers "F.Cu" "B.Cu") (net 2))
 (segment (start 142.33 73.53) (end 140.85 72.05) (width 0.2) (layer "B.Cu") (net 2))
 (segment (start 139.365686 74.25) (end 141.73 74.25) (width 0.2) (layer "B.Cu") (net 2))
 (segment (start 140.5 65.65) (end 136.75 69.4) (width 0.2) (layer "B.Cu") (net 2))
 (segment (start 123.746346 73.45) (end 123.526346 73.23) (width 0.2) (layer "B.Cu") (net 2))
 (segment (start 121.9 72.35) (end 121.9 70.45) (width 0.2) (layer "B.Cu") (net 2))
 (segment (start 123.526346 73.23) (end 122.78 73.23) (width 0.2) (layer "B.Cu") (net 2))
 (segment (start 142.45 73.53) (end 142.33 73.53) (width 0.2) (layer "B.Cu") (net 2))
 (segment (start 141.73 74.25) (end 142.45 73.53) (width 0.2) (layer "B.Cu") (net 2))
 (segment (start 139.365686 74.25) (end 138.565686 73.45) (width 0.2) (layer "B.Cu") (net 2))
 (segment (start 157.65 73.53) (end 142.45 73.53) (width 0.2) (layer "B.Cu") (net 2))
 (segment (start 138.565686 73.45) (end 123.746346 73.45) (width 0.2) (layer "B.Cu") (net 2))
 (segment (start 122.78 73.23) (end 121.9 72.35) (width 0.2) (layer "B.Cu") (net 2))
 (segment (start 136.75 69.4) (end 136.35 69.4) (width 0.2) (layer "B.Cu") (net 2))
 (segment (start 121.9 70.45) (end 123.05 69.3) (width 0.2) (layer "B.Cu") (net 2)))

